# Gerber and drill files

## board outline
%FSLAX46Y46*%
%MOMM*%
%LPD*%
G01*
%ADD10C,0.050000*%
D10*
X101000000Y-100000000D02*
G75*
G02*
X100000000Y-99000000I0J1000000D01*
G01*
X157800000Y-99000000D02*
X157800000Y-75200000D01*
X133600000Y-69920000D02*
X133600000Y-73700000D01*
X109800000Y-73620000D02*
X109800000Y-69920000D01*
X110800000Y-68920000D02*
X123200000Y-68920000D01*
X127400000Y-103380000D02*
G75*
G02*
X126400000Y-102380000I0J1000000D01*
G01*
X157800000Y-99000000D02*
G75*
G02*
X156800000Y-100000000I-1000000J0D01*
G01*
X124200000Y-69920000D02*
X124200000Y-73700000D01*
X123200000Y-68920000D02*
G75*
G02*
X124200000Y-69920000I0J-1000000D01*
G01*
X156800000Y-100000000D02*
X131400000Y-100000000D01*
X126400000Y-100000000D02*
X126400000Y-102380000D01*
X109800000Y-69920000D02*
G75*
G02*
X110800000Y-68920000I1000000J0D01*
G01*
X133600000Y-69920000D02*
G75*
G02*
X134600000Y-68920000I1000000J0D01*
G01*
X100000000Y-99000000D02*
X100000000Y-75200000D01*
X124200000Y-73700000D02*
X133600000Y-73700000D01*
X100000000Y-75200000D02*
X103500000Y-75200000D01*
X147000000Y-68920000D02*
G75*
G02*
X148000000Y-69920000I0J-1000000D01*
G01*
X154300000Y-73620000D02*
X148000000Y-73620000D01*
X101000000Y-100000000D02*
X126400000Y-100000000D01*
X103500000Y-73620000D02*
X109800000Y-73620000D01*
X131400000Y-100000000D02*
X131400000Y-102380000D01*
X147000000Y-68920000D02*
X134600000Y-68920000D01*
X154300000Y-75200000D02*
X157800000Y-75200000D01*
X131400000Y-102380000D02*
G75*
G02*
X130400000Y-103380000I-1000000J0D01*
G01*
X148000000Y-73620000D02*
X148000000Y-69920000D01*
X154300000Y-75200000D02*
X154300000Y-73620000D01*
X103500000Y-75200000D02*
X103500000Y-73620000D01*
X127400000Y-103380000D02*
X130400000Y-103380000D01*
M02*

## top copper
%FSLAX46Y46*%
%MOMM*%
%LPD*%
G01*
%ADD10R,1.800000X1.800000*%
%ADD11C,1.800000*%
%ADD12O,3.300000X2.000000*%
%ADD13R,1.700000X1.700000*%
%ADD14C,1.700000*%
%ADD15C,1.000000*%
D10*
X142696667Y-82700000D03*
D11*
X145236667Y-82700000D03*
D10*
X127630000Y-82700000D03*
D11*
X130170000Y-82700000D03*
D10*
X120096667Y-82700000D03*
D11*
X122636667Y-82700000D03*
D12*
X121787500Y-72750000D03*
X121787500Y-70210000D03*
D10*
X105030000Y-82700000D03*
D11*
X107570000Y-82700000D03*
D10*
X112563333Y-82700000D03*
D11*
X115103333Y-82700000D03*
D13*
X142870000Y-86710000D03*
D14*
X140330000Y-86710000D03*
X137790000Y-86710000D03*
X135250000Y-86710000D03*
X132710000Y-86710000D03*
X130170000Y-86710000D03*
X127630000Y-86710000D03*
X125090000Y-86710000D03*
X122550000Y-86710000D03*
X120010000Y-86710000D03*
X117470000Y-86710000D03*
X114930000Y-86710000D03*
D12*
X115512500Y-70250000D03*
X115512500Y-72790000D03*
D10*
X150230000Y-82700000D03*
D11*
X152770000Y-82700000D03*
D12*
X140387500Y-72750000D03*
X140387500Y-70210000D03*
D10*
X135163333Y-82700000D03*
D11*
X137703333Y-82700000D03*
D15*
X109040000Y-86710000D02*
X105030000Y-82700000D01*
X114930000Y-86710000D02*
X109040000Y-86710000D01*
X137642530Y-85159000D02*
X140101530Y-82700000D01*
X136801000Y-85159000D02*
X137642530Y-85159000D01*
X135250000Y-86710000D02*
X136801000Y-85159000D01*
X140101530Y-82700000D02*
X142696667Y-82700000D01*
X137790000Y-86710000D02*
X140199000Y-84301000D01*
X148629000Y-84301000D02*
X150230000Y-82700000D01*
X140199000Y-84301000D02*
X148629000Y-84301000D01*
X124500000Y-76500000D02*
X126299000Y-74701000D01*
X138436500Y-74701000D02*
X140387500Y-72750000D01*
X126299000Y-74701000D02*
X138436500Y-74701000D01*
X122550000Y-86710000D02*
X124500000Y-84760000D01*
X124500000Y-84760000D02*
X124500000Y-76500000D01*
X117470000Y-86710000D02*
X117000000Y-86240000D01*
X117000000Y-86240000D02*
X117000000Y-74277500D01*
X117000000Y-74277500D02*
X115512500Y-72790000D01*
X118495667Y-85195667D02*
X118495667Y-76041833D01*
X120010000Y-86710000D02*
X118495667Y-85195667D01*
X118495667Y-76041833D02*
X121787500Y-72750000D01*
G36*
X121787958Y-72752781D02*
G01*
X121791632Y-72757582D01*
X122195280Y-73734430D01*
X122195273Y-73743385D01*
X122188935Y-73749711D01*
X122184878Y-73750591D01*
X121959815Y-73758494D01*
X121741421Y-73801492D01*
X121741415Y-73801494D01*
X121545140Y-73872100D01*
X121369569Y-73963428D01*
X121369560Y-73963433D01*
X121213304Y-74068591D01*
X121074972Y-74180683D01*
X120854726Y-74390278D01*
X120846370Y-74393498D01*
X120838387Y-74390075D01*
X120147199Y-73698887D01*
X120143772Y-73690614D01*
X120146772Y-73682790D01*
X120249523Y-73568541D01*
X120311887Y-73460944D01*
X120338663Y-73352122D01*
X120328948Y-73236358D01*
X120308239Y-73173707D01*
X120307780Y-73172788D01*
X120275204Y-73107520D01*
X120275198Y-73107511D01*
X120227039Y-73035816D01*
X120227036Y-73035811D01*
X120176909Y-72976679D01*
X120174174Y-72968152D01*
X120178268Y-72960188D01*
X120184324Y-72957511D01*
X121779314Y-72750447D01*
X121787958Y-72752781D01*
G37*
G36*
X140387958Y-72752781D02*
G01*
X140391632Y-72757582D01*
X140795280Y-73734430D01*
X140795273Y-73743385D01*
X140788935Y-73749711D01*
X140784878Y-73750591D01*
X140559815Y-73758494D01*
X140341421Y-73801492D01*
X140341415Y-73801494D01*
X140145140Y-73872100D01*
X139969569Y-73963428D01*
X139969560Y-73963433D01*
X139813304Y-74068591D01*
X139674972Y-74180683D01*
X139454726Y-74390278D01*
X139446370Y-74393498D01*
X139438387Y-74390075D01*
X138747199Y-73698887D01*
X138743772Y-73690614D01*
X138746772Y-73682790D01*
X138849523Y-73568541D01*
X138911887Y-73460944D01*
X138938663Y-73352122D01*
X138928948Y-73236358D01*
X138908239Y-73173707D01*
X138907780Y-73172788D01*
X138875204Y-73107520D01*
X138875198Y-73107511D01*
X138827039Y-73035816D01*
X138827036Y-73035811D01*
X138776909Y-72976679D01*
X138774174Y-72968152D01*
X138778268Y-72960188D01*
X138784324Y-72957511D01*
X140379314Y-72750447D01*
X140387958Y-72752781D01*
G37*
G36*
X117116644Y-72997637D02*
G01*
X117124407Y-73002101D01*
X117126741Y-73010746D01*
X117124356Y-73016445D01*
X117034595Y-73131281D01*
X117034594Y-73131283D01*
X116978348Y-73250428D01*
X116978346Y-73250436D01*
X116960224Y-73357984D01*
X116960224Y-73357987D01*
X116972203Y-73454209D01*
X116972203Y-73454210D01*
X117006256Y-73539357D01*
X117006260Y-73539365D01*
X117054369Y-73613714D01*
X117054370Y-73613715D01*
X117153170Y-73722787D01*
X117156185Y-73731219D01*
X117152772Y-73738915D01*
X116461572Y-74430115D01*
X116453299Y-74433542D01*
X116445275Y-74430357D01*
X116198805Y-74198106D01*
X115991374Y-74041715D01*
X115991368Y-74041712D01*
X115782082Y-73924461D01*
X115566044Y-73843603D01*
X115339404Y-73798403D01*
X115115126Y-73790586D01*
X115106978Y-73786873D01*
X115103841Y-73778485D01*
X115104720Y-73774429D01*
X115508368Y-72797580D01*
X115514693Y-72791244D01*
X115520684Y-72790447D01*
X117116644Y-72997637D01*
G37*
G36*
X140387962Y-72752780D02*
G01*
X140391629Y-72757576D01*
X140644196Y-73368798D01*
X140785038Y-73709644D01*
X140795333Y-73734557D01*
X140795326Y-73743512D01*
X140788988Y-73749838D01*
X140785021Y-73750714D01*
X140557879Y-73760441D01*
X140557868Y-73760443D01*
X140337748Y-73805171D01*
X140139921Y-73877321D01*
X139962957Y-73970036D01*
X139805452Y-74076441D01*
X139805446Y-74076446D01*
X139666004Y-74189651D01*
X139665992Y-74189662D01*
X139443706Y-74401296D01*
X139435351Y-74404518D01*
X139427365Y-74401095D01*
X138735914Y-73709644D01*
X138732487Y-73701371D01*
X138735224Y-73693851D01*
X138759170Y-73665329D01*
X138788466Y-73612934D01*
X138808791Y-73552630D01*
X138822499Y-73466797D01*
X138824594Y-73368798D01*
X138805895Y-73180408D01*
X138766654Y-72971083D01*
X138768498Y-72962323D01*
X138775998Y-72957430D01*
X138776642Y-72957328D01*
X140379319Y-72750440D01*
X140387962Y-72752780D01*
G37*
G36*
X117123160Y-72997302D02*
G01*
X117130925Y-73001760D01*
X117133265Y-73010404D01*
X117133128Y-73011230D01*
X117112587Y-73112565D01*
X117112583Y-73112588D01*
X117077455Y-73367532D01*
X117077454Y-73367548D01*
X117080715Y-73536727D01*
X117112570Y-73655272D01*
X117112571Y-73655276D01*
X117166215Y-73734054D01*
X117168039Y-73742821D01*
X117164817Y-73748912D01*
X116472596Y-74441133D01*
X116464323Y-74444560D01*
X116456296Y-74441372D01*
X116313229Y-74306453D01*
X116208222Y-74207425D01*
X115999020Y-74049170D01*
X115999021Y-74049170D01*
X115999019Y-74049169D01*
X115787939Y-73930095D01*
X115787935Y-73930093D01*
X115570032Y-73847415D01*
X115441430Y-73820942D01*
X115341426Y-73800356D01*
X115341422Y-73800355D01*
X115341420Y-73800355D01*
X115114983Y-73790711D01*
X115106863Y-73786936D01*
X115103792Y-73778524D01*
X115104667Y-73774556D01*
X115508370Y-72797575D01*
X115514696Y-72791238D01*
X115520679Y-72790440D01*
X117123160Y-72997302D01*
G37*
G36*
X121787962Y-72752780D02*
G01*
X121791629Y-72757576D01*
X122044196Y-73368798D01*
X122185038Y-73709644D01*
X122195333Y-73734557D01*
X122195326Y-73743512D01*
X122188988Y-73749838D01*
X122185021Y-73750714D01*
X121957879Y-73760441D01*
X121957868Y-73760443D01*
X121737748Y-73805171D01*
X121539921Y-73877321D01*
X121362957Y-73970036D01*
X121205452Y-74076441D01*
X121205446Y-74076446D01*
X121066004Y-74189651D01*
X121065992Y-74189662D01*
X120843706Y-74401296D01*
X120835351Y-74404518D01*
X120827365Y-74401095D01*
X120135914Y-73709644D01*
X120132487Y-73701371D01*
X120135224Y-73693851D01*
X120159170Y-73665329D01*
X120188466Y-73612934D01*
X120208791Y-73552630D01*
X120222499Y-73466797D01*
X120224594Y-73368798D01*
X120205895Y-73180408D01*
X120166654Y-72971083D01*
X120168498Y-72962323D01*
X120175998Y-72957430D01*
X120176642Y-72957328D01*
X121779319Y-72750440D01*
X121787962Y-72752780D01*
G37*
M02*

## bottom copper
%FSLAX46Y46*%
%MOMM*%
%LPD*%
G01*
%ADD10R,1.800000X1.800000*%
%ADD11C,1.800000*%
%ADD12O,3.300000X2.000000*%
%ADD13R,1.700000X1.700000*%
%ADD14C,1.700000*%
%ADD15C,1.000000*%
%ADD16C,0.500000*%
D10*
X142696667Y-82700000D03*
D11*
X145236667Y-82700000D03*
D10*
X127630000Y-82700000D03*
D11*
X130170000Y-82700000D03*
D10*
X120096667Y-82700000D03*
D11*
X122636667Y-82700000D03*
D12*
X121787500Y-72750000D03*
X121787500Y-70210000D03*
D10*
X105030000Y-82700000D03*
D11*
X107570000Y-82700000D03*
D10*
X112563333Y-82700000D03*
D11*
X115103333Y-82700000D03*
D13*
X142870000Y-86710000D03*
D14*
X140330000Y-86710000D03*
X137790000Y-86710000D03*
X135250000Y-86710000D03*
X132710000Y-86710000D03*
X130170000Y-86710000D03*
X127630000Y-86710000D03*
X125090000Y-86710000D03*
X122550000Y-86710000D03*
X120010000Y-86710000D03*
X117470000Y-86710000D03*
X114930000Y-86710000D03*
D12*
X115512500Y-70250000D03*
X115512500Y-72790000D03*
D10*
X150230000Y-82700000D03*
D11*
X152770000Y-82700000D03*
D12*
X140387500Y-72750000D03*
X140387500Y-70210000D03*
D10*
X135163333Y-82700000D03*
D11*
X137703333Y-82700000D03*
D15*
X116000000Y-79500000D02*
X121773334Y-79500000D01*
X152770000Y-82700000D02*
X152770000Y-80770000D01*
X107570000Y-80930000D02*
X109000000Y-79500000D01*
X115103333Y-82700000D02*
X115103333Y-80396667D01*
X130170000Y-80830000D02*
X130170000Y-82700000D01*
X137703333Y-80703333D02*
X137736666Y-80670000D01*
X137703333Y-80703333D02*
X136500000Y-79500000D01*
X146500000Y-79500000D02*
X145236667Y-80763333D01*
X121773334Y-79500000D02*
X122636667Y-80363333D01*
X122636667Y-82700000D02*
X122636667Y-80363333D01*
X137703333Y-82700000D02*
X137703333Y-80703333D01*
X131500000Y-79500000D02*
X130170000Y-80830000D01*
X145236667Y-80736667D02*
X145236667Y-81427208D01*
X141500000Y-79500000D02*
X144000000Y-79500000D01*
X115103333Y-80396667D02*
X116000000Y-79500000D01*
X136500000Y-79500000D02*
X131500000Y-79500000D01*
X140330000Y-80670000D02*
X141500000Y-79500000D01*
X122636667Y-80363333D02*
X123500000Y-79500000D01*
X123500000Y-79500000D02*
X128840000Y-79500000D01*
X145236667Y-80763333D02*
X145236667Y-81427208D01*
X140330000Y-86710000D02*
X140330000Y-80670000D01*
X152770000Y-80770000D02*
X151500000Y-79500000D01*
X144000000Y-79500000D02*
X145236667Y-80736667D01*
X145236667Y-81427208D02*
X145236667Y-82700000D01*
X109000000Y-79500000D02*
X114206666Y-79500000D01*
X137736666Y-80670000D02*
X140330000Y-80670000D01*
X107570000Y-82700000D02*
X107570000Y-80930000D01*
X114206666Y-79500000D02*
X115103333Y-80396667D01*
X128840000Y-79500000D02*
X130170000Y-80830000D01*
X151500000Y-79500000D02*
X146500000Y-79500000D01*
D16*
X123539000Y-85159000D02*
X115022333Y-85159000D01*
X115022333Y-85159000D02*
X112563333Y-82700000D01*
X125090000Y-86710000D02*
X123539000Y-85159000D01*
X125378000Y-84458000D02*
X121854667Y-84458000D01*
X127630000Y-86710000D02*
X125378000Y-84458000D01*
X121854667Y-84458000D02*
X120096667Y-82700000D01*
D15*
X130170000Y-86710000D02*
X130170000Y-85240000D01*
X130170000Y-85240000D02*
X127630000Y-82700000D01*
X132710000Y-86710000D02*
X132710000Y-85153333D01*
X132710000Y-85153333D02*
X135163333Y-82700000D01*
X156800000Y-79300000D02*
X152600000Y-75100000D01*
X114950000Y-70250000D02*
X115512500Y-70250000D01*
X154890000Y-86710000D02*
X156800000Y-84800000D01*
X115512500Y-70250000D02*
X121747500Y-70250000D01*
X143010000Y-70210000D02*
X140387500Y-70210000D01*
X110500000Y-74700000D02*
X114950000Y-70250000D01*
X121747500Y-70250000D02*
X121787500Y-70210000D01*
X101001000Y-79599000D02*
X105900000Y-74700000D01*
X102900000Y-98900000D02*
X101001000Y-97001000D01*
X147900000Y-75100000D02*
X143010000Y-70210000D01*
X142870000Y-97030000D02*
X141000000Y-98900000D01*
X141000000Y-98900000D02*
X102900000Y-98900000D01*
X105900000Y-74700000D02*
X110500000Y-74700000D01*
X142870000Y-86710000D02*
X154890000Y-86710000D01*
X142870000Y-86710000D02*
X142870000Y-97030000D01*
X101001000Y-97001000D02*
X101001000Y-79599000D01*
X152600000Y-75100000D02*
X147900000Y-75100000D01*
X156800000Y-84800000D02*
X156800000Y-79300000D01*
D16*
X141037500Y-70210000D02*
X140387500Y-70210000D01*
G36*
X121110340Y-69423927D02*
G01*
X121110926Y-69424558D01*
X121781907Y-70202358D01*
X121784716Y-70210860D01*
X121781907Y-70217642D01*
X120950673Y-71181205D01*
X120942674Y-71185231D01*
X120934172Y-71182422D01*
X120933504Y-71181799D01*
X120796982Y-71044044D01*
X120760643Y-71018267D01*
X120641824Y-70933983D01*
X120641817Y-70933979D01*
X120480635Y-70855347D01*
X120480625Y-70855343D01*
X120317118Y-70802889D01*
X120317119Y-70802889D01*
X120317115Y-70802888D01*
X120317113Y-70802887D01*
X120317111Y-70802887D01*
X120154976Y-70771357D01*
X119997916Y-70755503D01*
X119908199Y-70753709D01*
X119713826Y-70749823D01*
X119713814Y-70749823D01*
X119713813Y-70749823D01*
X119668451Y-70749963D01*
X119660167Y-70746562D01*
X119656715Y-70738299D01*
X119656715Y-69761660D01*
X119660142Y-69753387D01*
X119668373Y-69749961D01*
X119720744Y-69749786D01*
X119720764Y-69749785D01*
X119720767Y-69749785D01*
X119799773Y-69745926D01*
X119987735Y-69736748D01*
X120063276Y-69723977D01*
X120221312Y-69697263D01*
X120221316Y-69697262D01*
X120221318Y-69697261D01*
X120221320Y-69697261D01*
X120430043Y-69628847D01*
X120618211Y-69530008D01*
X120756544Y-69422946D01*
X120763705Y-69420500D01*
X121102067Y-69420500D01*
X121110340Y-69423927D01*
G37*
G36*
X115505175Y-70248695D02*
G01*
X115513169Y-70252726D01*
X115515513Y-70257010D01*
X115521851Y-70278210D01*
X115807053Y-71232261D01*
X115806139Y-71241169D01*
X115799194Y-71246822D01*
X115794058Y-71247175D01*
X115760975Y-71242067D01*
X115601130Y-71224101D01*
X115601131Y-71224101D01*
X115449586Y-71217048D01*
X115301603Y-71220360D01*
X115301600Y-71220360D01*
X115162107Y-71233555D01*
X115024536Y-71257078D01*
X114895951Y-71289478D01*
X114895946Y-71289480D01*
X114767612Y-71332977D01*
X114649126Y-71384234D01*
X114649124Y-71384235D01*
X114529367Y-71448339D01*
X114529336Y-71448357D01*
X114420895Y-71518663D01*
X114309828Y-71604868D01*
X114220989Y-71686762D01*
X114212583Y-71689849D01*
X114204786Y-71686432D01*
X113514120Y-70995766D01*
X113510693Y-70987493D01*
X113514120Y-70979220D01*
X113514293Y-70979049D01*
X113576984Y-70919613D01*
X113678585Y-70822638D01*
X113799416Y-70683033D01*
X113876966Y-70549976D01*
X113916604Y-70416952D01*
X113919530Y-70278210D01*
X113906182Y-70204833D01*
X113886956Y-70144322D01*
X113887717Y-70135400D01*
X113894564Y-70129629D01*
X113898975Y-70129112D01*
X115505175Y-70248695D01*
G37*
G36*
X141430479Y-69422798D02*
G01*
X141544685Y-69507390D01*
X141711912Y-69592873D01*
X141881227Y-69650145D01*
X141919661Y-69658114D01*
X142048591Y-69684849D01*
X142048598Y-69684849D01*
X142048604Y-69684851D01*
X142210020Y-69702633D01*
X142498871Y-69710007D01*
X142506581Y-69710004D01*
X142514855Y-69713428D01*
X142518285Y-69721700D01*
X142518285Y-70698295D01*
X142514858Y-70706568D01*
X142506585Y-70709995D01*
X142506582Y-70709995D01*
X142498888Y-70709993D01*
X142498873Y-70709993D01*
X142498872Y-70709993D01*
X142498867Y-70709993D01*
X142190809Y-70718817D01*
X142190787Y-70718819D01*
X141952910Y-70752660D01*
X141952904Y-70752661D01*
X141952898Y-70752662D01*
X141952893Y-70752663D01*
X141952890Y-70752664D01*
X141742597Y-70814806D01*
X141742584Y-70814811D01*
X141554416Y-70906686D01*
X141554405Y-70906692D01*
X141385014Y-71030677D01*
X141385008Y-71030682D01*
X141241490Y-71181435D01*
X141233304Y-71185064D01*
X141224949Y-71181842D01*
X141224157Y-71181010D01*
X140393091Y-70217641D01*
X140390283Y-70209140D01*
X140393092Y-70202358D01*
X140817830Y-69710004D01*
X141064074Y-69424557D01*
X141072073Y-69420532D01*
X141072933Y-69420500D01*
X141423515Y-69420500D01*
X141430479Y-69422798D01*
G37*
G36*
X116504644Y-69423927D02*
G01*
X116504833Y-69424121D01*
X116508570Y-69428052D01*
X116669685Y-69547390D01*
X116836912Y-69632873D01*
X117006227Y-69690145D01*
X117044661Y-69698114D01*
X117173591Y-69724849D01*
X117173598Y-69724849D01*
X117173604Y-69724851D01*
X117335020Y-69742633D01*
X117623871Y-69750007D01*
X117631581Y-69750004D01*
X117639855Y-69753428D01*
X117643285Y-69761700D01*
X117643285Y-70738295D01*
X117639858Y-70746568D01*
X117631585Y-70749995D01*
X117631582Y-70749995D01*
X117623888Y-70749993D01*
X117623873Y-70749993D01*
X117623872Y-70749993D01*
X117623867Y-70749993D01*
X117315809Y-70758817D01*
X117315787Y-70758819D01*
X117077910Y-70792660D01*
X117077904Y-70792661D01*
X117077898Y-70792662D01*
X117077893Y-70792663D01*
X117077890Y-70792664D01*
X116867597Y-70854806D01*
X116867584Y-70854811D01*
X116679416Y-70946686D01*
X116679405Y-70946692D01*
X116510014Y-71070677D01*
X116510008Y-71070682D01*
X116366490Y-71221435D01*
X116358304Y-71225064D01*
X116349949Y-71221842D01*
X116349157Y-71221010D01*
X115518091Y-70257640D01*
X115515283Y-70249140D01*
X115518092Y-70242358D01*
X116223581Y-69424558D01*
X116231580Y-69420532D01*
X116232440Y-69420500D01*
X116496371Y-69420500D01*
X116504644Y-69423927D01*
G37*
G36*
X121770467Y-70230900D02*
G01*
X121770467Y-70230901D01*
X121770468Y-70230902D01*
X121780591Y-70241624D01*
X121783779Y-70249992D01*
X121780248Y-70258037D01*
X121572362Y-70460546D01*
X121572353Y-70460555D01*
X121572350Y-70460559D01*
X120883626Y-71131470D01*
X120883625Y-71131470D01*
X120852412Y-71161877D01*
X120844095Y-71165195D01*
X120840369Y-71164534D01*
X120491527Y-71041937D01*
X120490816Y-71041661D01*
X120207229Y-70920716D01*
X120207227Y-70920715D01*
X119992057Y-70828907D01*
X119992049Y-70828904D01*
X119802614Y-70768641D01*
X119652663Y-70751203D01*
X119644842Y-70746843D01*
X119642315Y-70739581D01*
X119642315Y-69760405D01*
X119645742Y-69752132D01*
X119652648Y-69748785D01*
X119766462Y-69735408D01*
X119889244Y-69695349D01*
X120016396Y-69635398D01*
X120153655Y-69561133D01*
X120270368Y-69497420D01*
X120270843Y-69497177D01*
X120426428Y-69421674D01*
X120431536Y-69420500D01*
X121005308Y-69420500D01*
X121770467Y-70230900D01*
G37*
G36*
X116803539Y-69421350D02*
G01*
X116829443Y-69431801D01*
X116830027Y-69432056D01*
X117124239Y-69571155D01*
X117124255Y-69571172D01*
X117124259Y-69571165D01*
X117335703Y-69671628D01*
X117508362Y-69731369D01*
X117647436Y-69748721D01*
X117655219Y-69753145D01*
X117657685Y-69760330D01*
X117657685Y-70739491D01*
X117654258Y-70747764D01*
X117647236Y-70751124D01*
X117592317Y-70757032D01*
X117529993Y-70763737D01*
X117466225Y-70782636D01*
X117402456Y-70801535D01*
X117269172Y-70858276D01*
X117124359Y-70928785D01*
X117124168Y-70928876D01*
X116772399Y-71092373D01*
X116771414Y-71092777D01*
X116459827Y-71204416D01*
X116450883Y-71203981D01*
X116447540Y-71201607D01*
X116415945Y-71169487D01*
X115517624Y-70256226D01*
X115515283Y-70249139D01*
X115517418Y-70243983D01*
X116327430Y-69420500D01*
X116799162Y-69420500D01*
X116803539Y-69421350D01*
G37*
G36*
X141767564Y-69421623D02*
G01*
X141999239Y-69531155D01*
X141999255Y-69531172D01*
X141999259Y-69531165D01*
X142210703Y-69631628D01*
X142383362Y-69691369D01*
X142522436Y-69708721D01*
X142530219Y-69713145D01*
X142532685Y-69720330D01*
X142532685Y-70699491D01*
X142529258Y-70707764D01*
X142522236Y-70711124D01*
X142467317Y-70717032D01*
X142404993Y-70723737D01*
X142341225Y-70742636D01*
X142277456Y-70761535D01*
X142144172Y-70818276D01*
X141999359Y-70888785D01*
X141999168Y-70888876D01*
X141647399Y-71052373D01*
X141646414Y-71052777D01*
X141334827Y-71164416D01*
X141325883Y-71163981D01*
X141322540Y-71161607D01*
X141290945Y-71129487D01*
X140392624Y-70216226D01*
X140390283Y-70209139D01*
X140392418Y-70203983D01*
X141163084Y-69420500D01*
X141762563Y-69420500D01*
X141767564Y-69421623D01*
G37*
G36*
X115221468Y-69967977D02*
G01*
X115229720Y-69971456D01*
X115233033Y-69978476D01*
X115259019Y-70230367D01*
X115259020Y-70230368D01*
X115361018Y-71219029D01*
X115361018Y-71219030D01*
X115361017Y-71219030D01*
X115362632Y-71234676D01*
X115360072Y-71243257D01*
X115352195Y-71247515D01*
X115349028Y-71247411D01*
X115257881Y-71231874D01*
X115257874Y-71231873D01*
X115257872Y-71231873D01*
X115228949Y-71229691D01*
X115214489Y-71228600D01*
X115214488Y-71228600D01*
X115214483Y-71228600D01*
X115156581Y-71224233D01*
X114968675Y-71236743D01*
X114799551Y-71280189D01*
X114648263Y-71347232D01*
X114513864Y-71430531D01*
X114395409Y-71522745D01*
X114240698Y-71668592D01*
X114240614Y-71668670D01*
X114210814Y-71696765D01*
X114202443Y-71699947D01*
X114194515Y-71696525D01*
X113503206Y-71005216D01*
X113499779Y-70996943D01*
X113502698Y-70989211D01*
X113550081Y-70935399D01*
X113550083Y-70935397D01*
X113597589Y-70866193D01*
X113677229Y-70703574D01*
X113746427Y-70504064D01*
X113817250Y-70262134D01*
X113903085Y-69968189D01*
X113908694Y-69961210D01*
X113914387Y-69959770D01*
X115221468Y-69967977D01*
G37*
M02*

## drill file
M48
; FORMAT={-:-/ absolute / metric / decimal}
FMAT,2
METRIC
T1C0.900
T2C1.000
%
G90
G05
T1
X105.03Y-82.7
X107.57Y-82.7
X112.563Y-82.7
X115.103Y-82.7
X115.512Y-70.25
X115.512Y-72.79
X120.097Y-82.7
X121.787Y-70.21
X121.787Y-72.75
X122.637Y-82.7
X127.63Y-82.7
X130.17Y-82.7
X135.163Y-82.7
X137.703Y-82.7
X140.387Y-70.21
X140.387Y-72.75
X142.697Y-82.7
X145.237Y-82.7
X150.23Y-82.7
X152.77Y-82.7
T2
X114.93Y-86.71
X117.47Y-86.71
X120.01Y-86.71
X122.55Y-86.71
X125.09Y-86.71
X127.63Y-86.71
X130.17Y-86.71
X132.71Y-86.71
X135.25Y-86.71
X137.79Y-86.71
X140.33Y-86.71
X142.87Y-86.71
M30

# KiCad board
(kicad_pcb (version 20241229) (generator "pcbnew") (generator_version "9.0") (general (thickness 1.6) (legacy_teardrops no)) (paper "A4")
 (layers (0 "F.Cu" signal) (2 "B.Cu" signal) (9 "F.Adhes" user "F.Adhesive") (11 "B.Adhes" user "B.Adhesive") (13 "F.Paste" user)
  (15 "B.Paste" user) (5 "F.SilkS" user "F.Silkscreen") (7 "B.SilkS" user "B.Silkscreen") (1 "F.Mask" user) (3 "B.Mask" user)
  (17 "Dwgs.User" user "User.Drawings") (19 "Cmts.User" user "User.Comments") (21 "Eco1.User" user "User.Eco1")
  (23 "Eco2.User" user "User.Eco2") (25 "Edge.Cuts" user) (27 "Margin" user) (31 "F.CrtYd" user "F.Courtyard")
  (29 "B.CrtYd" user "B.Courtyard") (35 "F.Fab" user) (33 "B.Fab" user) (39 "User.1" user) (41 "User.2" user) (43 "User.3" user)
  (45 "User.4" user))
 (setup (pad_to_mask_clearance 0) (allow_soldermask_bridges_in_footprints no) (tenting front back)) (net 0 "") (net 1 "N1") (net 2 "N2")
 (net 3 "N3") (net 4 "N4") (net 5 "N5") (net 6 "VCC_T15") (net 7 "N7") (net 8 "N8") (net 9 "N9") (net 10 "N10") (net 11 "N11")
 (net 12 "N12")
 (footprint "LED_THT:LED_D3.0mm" (layer "F.Cu") (at 142.696667 82.7)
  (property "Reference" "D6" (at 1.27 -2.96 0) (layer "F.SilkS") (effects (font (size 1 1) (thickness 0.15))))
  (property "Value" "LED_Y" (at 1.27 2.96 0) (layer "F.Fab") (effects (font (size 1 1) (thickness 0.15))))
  (pad "1" thru_hole rect (at 0 0) (size 1.8 1.8) (drill 0.9) (layers "*.Cu" "*.Mask") (remove_unused_layers no) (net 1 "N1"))
  (pad "2" thru_hole circle (at 2.54 0) (size 1.8 1.8) (drill 0.9) (layers "*.Cu" "*.Mask") (remove_unused_layers no) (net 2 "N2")))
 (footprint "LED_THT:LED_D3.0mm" (layer "F.Cu") (at 127.63 82.7)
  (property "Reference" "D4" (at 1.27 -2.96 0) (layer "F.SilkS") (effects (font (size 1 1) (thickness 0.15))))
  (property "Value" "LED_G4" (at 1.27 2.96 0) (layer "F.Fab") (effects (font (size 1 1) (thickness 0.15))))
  (pad "1" thru_hole rect (at 0 0) (size 1.8 1.8) (drill 0.9) (layers "*.Cu" "*.Mask") (remove_unused_layers no) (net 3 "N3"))
  (pad "2" thru_hole circle (at 2.54 0) (size 1.8 1.8) (drill 0.9) (layers "*.Cu" "*.Mask") (remove_unused_layers no) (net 2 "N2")))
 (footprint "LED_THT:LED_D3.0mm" (layer "F.Cu") (at 120.096667 82.7)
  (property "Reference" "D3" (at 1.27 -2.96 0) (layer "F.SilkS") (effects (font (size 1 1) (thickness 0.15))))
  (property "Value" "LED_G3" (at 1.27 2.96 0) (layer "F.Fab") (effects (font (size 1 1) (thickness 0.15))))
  (pad "1" thru_hole rect (at 0 0) (size 1.8 1.8) (drill 0.9) (layers "*.Cu" "*.Mask") (remove_unused_layers no) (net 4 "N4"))
  (pad "2" thru_hole circle (at 2.54 0) (size 1.8 1.8) (drill 0.9) (layers "*.Cu" "*.Mask") (remove_unused_layers no) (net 2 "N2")))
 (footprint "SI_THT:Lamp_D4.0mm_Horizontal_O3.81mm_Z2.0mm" (layer "F.Cu") (at 121.7875 72.75 90)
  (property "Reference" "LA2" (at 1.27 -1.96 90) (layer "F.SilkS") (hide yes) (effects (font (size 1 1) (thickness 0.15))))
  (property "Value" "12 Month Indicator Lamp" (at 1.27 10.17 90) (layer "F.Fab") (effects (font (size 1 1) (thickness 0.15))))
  (pad "1" thru_hole oval (at 0 0 90) (size 2 3.3) (drill 0.9) (layers "*.Cu" "*.Mask") (remove_unused_layers no) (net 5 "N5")
   (teardrops (best_length_ratio 0.3) (max_length 0.5) (best_width_ratio 1) (max_width 2) (curved_edges yes) (filter_ratio 0.9)
    (enabled yes) (allow_two_segments yes) (prefer_zone_connections yes)))
  (pad "2" thru_hole oval (at 2.54 0 90) (size 2 3.3) (drill 0.9) (layers "*.Cu" "*.Mask") (remove_unused_layers no) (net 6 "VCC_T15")
   (teardrops (best_length_ratio 0.3) (max_length 0.5) (best_width_ratio 1) (max_width 2) (curved_edges yes) (filter_ratio 0.9)
    (enabled yes) (allow_two_segments yes) (prefer_zone_connections yes))))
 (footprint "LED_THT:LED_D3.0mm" (layer "F.Cu") (at 105.03 82.7)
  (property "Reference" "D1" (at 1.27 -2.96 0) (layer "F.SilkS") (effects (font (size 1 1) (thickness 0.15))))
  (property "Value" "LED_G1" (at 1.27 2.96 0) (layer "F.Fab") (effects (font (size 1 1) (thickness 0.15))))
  (pad "1" thru_hole rect (at 0 0) (size 1.8 1.8) (drill 0.9) (layers "*.Cu" "*.Mask") (remove_unused_layers no) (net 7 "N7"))
  (pad "2" thru_hole circle (at 2.54 0) (size 1.8 1.8) (drill 0.9) (layers "*.Cu" "*.Mask") (remove_unused_layers no) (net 2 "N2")))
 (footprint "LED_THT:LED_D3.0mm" (layer "F.Cu") (at 112.563333 82.7)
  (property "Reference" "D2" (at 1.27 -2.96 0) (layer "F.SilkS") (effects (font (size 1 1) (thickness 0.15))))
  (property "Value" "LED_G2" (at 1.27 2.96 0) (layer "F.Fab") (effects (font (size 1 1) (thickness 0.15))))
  (pad "1" thru_hole rect (at 0 0) (size 1.8 1.8) (drill 0.9) (layers "*.Cu" "*.Mask") (remove_unused_layers no) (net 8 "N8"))
  (pad "2" thru_hole circle (at 2.54 0) (size 1.8 1.8) (drill 0.9) (layers "*.Cu" "*.Mask") (remove_unused_layers no) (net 2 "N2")))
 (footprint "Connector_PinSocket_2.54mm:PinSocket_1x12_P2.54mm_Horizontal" (layer "F.Cu") (at 114.87 86.71 90)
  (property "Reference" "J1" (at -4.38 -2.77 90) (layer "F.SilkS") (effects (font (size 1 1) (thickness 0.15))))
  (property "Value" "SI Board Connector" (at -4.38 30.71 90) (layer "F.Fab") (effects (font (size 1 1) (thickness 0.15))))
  (pad "1" thru_hole rect (at 0 28 90) (size 1.7 1.7) (drill 1) (layers "*.Cu" "*.Mask") (remove_unused_layers no) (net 6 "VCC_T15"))
  (pad "2" thru_hole circle (at 0 25.46 90) (size 1.7 1.7) (drill 1) (layers "*.Cu" "*.Mask") (remove_unused_layers no) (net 2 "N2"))
  (pad "3" thru_hole circle (at 0 22.92 90) (size 1.7 1.7) (drill 1) (layers "*.Cu" "*.Mask") (remove_unused_layers no) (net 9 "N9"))
  (pad "4" thru_hole circle (at 0 20.38 90) (size 1.7 1.7) (drill 1) (layers "*.Cu" "*.Mask") (remove_unused_layers no) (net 1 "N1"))
  (pad "5" thru_hole circle (at 0 17.84 90) (size 1.7 1.7) (drill 1) (layers "*.Cu" "*.Mask") (remove_unused_layers no) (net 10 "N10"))
  (pad "6" thru_hole circle (at 0 15.3 90) (size 1.7 1.7) (drill 1) (layers "*.Cu" "*.Mask") (remove_unused_layers no) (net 3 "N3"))
  (pad "7" thru_hole circle (at 0 12.76 90) (size 1.7 1.7) (drill 1) (layers "*.Cu" "*.Mask") (remove_unused_layers no) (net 4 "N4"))
  (pad "8" thru_hole circle (at 0 10.22 90) (size 1.7 1.7) (drill 1) (layers "*.Cu" "*.Mask") (remove_unused_layers no) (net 8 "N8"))
  (pad "9" thru_hole circle (at 0 7.68 90) (size 1.7 1.7) (drill 1) (layers "*.Cu" "*.Mask") (remove_unused_layers no) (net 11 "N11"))
  (pad "10" thru_hole circle (at 0 5.14 90) (size 1.7 1.7) (drill 1) (layers "*.Cu" "*.Mask") (remove_unused_layers no) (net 5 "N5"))
  (pad "11" thru_hole circle (at 0 2.6 90) (size 1.7 1.7) (drill 1) (layers "*.Cu" "*.Mask") (remove_unused_layers no) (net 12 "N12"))
  (pad "12" thru_hole circle (at 0 0.06 90) (size 1.7 1.7) (drill 1) (layers "*.Cu" "*.Mask") (remove_unused_layers no) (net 7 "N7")))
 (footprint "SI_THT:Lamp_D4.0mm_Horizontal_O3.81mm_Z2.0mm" (layer "F.Cu") (at 115.5125 70.25 -90)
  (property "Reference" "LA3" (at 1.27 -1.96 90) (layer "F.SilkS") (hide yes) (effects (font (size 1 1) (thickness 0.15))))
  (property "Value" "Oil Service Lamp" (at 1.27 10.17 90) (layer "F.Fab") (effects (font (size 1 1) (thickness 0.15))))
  (pad "1" thru_hole oval (at 0 0 270) (size 2 3.3) (drill 0.9) (layers "*.Cu" "*.Mask") (remove_unused_layers no) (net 6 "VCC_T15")
   (teardrops (best_length_ratio 0.3) (max_length 0.5) (best_width_ratio 1) (max_width 2) (curved_edges yes) (filter_ratio 0.9)
    (enabled yes) (allow_two_segments yes) (prefer_zone_connections yes)))
  (pad "2" thru_hole oval (at 2.54 0 270) (size 2 3.3) (drill 0.9) (layers "*.Cu" "*.Mask") (remove_unused_layers no) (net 12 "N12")
   (teardrops (best_length_ratio 0.3) (max_length 0.5) (best_width_ratio 1) (max_width 2) (curved_edges yes) (filter_ratio 0.9)
    (enabled yes) (allow_two_segments yes) (prefer_zone_connections yes))))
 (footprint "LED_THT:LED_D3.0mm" (layer "F.Cu") (at 150.23 82.7)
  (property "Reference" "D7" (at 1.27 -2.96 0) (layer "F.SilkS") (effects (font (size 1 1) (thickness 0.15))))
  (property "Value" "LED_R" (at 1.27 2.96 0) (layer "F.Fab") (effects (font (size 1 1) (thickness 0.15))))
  (pad "1" thru_hole rect (at 0 0) (size 1.8 1.8) (drill 0.9) (layers "*.Cu" "*.Mask") (remove_unused_layers no) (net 9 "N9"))
  (pad "2" thru_hole circle (at 2.54 0) (size 1.8 1.8) (drill 0.9) (layers "*.Cu" "*.Mask") (remove_unused_layers no) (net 2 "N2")))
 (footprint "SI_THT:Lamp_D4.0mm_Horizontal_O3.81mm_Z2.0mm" (layer "F.Cu") (at 140.3875 72.75 90)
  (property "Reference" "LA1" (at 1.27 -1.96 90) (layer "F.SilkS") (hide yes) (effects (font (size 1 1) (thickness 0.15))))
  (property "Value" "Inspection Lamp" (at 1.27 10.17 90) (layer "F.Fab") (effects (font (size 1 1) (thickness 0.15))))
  (pad "1" thru_hole oval (at 0 0 90) (size 2 3.3) (drill 0.9) (layers "*.Cu" "*.Mask") (remove_unused_layers no) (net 11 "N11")
   (teardrops (best_length_ratio 0.3) (max_length 0.5) (best_width_ratio 1) (max_width 2) (curved_edges yes) (filter_ratio 0.9)
    (enabled yes) (allow_two_segments yes) (prefer_zone_connections yes)))
  (pad "2" thru_hole oval (at 2.54 0 90) (size 2 3.3) (drill 0.9) (layers "*.Cu" "*.Mask") (remove_unused_layers no) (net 6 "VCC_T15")
   (teardrops (best_length_ratio 0.3) (max_length 0.5) (best_width_ratio 1) (max_width 2) (curved_edges yes) (filter_ratio 0.9)
    (enabled yes) (allow_two_segments yes) (prefer_zone_connections yes))))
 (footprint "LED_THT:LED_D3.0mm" (layer "F.Cu") (at 135.163333 82.7)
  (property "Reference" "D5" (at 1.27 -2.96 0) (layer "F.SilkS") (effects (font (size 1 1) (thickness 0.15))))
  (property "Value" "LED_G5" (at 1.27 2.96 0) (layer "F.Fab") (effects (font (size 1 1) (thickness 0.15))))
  (pad "1" thru_hole rect (at 0 0) (size 1.8 1.8) (drill 0.9) (layers "*.Cu" "*.Mask") (remove_unused_layers no) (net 10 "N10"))
  (pad "2" thru_hole circle (at 2.54 0) (size 1.8 1.8) (drill 0.9) (layers "*.Cu" "*.Mask") (remove_unused_layers no) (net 2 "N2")))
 (gr_arc (start 101 100) (mid 100.292893 99.707107) (end 100 99) (stroke (width 0.05) (type default)) (layer "Edge.Cuts"))
 (gr_line (start 157.8 99) (end 157.8 75.2) (stroke (width 0.05) (type solid)) (layer "Edge.Cuts"))
 (gr_line (start 133.6 69.92) (end 133.6 73.7) (stroke (width 0.05) (type solid)) (layer "Edge.Cuts"))
 (gr_line (start 109.8 73.62) (end 109.8 69.92) (stroke (width 0.05) (type solid)) (layer "Edge.Cuts"))
 (gr_line (start 110.8 68.92) (end 123.2 68.92) (stroke (width 0.05) (type solid)) (layer "Edge.Cuts"))
 (gr_arc (start 127.4 103.38) (mid 126.692893 103.087107) (end 126.4 102.38) (stroke (width 0.05) (type default)) (layer "Edge.Cuts"))
 (gr_arc (start 157.8 99) (mid 157.507107 99.707107) (end 156.8 100) (stroke (width 0.05) (type default)) (layer "Edge.Cuts"))
 (gr_line (start 124.2 69.92) (end 124.2 73.7) (stroke (width 0.05) (type solid)) (layer "Edge.Cuts"))
 (gr_arc (start 123.2 68.92) (mid 123.907107 69.212893) (end 124.2 69.92) (stroke (width 0.05) (type default)) (layer "Edge.Cuts"))
 (gr_line (start 156.8 100) (end 131.4 100) (stroke (width 0.05) (type solid)) (layer "Edge.Cuts"))
 (gr_line (start 126.4 100) (end 126.4 102.38) (stroke (width 0.05) (type solid)) (layer "Edge.Cuts"))
 (gr_arc (start 109.8 69.92) (mid 110.092893 69.212893) (end 110.8 68.92) (stroke (width 0.05) (type default)) (layer "Edge.Cuts"))
 (gr_arc (start 133.6 69.92) (mid 133.892893 69.212893) (end 134.6 68.92) (stroke (width 0.05) (type default)) (layer "Edge.Cuts"))
 (gr_line (start 100 99) (end 100 75.2) (stroke (width 0.05) (type solid)) (layer "Edge.Cuts"))
 (gr_line (start 124.2 73.7) (end 133.6 73.7) (stroke (width 0.05) (type default)) (layer "Edge.Cuts"))
 (gr_line (start 100 75.2) (end 103.5 75.2) (stroke (width 0.05) (type solid)) (layer "Edge.Cuts"))
 (gr_arc (start 147 68.92) (mid 147.707107 69.212893) (end 148 69.92) (stroke (width 0.05) (type default)) (layer "Edge.Cuts"))
 (gr_line (start 154.3 73.62) (end 148 73.62) (stroke (width 0.05) (type solid)) (layer "Edge.Cuts"))
 (gr_line (start 101 100) (end 126.4 100) (stroke (width 0.05) (type solid)) (layer "Edge.Cuts"))
 (gr_line (start 103.5 73.62) (end 109.8 73.62) (stroke (width 0.05) (type solid)) (layer "Edge.Cuts"))
 (gr_line (start 131.4 100) (end 131.4 102.38) (stroke (width 0.05) (type solid)) (layer "Edge.Cuts"))
 (gr_line (start 147 68.92) (end 134.6 68.92) (stroke (width 0.05) (type solid)) (layer "Edge.Cuts"))
 (gr_line (start 154.3 75.2) (end 157.8 75.2) (stroke (width 0.05) (type solid)) (layer "Edge.Cuts"))
 (gr_arc (start 131.4 102.38) (mid 131.107107 103.087107) (end 130.4 103.38) (stroke (width 0.05) (type default)) (layer "Edge.Cuts"))
 (gr_line (start 148 73.62) (end 148 69.92) (stroke (width 0.05) (type solid)) (layer "Edge.Cuts"))
 (gr_line (start 154.3 75.2) (end 154.3 73.62) (stroke (width 0.05) (type solid)) (layer "Edge.Cuts"))
 (gr_line (start 103.5 75.2) (end 103.5 73.62) (stroke (width 0.05) (type solid)) (layer "Edge.Cuts"))
 (gr_line (start 127.4 103.38) (end 130.4 103.38) (stroke (width 0.05) (type solid)) (layer "Edge.Cuts"))
 (segment (start 116 79.5) (end 121.773334 79.5) (width 1) (layer "B.Cu") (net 2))
 (segment (start 152.77 82.7) (end 152.77 80.77) (width 1) (layer "B.Cu") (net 2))
 (segment (start 107.57 80.93) (end 109 79.5) (width 1) (layer "B.Cu") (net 2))
 (segment (start 115.103333 82.7) (end 115.103333 80.396667) (width 1) (layer "B.Cu") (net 2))
 (segment (start 130.17 80.83) (end 130.17 82.7) (width 1) (layer "B.Cu") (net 2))
 (segment (start 137.703333 80.703333) (end 137.736666 80.67) (width 1) (layer "B.Cu") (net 2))
 (segment (start 137.703333 80.703333) (end 136.5 79.5) (width 1) (layer "B.Cu") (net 2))
 (segment (start 146.5 79.5) (end 145.236667 80.763333) (width 1) (layer "B.Cu") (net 2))
 (segment (start 121.773334 79.5) (end 122.636667 80.363333) (width 1) (layer "B.Cu") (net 2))
 (segment (start 122.636667 82.7) (end 122.636667 80.363333) (width 1) (layer "B.Cu") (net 2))
 (segment (start 137.703333 82.7) (end 137.703333 80.703333) (width 1) (layer "B.Cu") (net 2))
 (segment (start 131.5 79.5) (end 130.17 80.83) (width 1) (layer "B.Cu") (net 2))
 (segment (start 145.236667 80.736667) (end 145.236667 81.427208) (width 1) (layer "B.Cu") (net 2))
 (segment (start 141.5 79.5) (end 144 79.5) (width 1) (layer "B.Cu") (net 2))
 (segment (start 115.103333 80.396667) (end 116 79.5) (width 1) (layer "B.Cu") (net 2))
 (segment (start 136.5 79.5) (end 131.5 79.5) (width 1) (layer "B.Cu") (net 2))
 (segment (start 140.33 80.67) (end 141.5 79.5) (width 1) (layer "B.Cu") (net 2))
 (segment (start 122.636667 80.363333) (end 123.5 79.5) (width 1) (layer "B.Cu") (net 2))
 (segment (start 123.5 79.5) (end 128.84 79.5) (width 1) (layer "B.Cu") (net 2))
 (segment (start 145.236667 80.763333) (end 145.236667 81.427208) (width 1) (layer "B.Cu") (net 2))
 (segment (start 140.33 86.71) (end 140.33 80.67) (width 1) (layer "B.Cu") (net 2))
 (segment (start 152.77 80.77) (end 151.5 79.5) (width 1) (layer "B.Cu") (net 2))
 (segment (start 144 79.5) (end 145.236667 80.736667) (width 1) (layer "B.Cu") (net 2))
 (segment (start 145.236667 81.427208) (end 145.236667 82.7) (width 1) (layer "B.Cu") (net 2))
 (segment (start 109 79.5) (end 114.206666 79.5) (width 1) (layer "B.Cu") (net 2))
 (segment (start 137.736666 80.67) (end 140.33 80.67) (width 1) (layer "B.Cu") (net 2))
 (segment (start 107.57 82.7) (end 107.57 80.93) (width 1) (layer "B.Cu") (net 2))
 (segment (start 114.206666 79.5) (end 115.103333 80.396667) (width 1) (layer "B.Cu") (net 2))
 (segment (start 128.84 79.5) (end 130.17 80.83) (width 1) (layer "B.Cu") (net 2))
 (segment (start 151.5 79.5) (end 146.5 79.5) (width 1) (layer "B.Cu") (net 2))
 (segment (start 109.04 86.71) (end 105.03 82.7) (width 1) (layer "F.Cu") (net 7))
 (segment (start 114.93 86.71) (end 109.04 86.71) (width 1) (layer "F.Cu") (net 7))
 (segment (start 123.539 85.159) (end 115.022333 85.159) (width 0.5) (layer "B.Cu") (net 8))
 (segment (start 115.022333 85.159) (end 112.563333 82.7) (width 0.5) (layer "B.Cu") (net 8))
 (segment (start 125.09 86.71) (end 123.539 85.159) (width 0.5) (layer "B.Cu") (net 8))
 (segment (start 125.378 84.458) (end 121.854667 84.458) (width 0.5) (layer "B.Cu") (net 4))
 (segment (start 127.63 86.71) (end 125.378 84.458) (width 0.5) (layer "B.Cu") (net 4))
 (segment (start 121.854667 84.458) (end 120.096667 82.7) (width 0.5) (layer "B.Cu") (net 4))
 (segment (start 130.17 86.71) (end 130.17 85.24) (width 1) (layer "B.Cu") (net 3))
 (segment (start 130.17 85.24) (end 127.63 82.7) (width 1) (layer "B.Cu") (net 3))
 (segment (start 132.71 86.71) (end 132.71 85.153333) (width 1) (layer "B.Cu") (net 10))
 (segment (start 132.71 85.153333) (end 135.163333 82.7) (width 1) (layer "B.Cu") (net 10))
 (segment (start 137.64253 85.159) (end 140.10153 82.7) (width 1) (layer "F.Cu") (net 1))
 (segment (start 136.801 85.159) (end 137.64253 85.159) (width 1) (layer "F.Cu") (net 1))
 (segment (start 135.25 86.71) (end 136.801 85.159) (width 1) (layer "F.Cu") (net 1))
 (segment (start 140.10153 82.7) (end 142.696667 82.7) (width 1) (layer "F.Cu") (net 1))
 (segment (start 137.79 86.71) (end 140.199 84.301) (width 1) (layer "F.Cu") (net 9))
 (segment (start 148.629 84.301) (end 150.23 82.7) (width 1) (layer "F.Cu") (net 9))
 (segment (start 140.199 84.301) (end 148.629 84.301) (width 1) (layer "F.Cu") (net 9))
 (segment (start 124.5 76.5) (end 126.299 74.701) (width 1) (layer "F.Cu") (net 11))
 (segment (start 138.4365 74.701) (end 140.3875 72.75) (width 1) (layer "F.Cu") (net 11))
 (segment (start 126.299 74.701) (end 138.4365 74.701) (width 1) (layer "F.Cu") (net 11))
 (segment (start 122.55 86.71) (end 124.5 84.76) (width 1) (layer "F.Cu") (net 11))
 (segment (start 124.5 84.76) (end 124.5 76.5) (width 1) (layer "F.Cu") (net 11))
 (segment (start 117.47 86.71) (end 117 86.24) (width 1) (layer "F.Cu") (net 12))
 (segment (start 117 86.24) (end 117 74.2775) (width 1) (layer "F.Cu") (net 12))
 (segment (start 117 74.2775) (end 115.5125 72.79) (width 1) (layer "F.Cu") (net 12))
 (segment (start 118.495667 85.195667) (end 118.495667 76.041833) (width 1) (layer "F.Cu") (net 5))
 (segment (start 120.01 86.71) (end 118.495667 85.195667) (width 1) (layer "F.Cu") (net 5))
 (segment (start 118.495667 76.041833) (end 121.7875 72.75) (width 1) (layer "F.Cu") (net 5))
 (segment (start 156.8 79.3) (end 152.6 75.1) (width 1) (layer "B.Cu") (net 6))
 (segment (start 114.95 70.25) (end 115.5125 70.25) (width 1) (layer "B.Cu") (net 6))
 (segment (start 154.89 86.71) (end 156.8 84.8) (width 1) (layer "B.Cu") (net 6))
 (segment (start 115.5125 70.25) (end 121.7475 70.25) (width 1) (layer "B.Cu") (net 6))
 (segment (start 143.01 70.21) (end 140.3875 70.21) (width 1) (layer "B.Cu") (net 6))
 (segment (start 110.5 74.7) (end 114.95 70.25) (width 1) (layer "B.Cu") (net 6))
 (segment (start 121.7475 70.25) (end 121.7875 70.21) (width 1) (layer "B.Cu") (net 6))
 (segment (start 101.001 79.599) (end 105.9 74.7) (width 1) (layer "B.Cu") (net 6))
 (segment (start 102.9 98.9) (end 101.001 97.001) (width 1) (layer "B.Cu") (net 6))
 (segment (start 147.9 75.1) (end 143.01 70.21) (width 1) (layer "B.Cu") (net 6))
 (segment (start 142.87 97.03) (end 141 98.9) (width 1) (layer "B.Cu") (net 6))
 (segment (start 141 98.9) (end 102.9 98.9) (width 1) (layer "B.Cu") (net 6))
 (segment (start 105.9 74.7) (end 110.5 74.7) (width 1) (layer "B.Cu") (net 6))
 (segment (start 142.87 86.71) (end 154.89 86.71) (width 1) (layer "B.Cu") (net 6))
 (segment (start 142.87 86.71) (end 142.87 97.03) (width 1) (layer "B.Cu") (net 6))
 (segment (start 101.001 97.001) (end 101.001 79.599) (width 1) (layer "B.Cu") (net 6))
 (segment (start 152.6 75.1) (end 147.9 75.1) (width 1) (layer "B.Cu") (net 6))
 (segment (start 156.8 84.8) (end 156.8 79.3) (width 1) (layer "B.Cu") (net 6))
 (segment (start 141.0375 70.21) (end 140.3875 70.21) (width 0.5) (layer "B.Cu") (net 6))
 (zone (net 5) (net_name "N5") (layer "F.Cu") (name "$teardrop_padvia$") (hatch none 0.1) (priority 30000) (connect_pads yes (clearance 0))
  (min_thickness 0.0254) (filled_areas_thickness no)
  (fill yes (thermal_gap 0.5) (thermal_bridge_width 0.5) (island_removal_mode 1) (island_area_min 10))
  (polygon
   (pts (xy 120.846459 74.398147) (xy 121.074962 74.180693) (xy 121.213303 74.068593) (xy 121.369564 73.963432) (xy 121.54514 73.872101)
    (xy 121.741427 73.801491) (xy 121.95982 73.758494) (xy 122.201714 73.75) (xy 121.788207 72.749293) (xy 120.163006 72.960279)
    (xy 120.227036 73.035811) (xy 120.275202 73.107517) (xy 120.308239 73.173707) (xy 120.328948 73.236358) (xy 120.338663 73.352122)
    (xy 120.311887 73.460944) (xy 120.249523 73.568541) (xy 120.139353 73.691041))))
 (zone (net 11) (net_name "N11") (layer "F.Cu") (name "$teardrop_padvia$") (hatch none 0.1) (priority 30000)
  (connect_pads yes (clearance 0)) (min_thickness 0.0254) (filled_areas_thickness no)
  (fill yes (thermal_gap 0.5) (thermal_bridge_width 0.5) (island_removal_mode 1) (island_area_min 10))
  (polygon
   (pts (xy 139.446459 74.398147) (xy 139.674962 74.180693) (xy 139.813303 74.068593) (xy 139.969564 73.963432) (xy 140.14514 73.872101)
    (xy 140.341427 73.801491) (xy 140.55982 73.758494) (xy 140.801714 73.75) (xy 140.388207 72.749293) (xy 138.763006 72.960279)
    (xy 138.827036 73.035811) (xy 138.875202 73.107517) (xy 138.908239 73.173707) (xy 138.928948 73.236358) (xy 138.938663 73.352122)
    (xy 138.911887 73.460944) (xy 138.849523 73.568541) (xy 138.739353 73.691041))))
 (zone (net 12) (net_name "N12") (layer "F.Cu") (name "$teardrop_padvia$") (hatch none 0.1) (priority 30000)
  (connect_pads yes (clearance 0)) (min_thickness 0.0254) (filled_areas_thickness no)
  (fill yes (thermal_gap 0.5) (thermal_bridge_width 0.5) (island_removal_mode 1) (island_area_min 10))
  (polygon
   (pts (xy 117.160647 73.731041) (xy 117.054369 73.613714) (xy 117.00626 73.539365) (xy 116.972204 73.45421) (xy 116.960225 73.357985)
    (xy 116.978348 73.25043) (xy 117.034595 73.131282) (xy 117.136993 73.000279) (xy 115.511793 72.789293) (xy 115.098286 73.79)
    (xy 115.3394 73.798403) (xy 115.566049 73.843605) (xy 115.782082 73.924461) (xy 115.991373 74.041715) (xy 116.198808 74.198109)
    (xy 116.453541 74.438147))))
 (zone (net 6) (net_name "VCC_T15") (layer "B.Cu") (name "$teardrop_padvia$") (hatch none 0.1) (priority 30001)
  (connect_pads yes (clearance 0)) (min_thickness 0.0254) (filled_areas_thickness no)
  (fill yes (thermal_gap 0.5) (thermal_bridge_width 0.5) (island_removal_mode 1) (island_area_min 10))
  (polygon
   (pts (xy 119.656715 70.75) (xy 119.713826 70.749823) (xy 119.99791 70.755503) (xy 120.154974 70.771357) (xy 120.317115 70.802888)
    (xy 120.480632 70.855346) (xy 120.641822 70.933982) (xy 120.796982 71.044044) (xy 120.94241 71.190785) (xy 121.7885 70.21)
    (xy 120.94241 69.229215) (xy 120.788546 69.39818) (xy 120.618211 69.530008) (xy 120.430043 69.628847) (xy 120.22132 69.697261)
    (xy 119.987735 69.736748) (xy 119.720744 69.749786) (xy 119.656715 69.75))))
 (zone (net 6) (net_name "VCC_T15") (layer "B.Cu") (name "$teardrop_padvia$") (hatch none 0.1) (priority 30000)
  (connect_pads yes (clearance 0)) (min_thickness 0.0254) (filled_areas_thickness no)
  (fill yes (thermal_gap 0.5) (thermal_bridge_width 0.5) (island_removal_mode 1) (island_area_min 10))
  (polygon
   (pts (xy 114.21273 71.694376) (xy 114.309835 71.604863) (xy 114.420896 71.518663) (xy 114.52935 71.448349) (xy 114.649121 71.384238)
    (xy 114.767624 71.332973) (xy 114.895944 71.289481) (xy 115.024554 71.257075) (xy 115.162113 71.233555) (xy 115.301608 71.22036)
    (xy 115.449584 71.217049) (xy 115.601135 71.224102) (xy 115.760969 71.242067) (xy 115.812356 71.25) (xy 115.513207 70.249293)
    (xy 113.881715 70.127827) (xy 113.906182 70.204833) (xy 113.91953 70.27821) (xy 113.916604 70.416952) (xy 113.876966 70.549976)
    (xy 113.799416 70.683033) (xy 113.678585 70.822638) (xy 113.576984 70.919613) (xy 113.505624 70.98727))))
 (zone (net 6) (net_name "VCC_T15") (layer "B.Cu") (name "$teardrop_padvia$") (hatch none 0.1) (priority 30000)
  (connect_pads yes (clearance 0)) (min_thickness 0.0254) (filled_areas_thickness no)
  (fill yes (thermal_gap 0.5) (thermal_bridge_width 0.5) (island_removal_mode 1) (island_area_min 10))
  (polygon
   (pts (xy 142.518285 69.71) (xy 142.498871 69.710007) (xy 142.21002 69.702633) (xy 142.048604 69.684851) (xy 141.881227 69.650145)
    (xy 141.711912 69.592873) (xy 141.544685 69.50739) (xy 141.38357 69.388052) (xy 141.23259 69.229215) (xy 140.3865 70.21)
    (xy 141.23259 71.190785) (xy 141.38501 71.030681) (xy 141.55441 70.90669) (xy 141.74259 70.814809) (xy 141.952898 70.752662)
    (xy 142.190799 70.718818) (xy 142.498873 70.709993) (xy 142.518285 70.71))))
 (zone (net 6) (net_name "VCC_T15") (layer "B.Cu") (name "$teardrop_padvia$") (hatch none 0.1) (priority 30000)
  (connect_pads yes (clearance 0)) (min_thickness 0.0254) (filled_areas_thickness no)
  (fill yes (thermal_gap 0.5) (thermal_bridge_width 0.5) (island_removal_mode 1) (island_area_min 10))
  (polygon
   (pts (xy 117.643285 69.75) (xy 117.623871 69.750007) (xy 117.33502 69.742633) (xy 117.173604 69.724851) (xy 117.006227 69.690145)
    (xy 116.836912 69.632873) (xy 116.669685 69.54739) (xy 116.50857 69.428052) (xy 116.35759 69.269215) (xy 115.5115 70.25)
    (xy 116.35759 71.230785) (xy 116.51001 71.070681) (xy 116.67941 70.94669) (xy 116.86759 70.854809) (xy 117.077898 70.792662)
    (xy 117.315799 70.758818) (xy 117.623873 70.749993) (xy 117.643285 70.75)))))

